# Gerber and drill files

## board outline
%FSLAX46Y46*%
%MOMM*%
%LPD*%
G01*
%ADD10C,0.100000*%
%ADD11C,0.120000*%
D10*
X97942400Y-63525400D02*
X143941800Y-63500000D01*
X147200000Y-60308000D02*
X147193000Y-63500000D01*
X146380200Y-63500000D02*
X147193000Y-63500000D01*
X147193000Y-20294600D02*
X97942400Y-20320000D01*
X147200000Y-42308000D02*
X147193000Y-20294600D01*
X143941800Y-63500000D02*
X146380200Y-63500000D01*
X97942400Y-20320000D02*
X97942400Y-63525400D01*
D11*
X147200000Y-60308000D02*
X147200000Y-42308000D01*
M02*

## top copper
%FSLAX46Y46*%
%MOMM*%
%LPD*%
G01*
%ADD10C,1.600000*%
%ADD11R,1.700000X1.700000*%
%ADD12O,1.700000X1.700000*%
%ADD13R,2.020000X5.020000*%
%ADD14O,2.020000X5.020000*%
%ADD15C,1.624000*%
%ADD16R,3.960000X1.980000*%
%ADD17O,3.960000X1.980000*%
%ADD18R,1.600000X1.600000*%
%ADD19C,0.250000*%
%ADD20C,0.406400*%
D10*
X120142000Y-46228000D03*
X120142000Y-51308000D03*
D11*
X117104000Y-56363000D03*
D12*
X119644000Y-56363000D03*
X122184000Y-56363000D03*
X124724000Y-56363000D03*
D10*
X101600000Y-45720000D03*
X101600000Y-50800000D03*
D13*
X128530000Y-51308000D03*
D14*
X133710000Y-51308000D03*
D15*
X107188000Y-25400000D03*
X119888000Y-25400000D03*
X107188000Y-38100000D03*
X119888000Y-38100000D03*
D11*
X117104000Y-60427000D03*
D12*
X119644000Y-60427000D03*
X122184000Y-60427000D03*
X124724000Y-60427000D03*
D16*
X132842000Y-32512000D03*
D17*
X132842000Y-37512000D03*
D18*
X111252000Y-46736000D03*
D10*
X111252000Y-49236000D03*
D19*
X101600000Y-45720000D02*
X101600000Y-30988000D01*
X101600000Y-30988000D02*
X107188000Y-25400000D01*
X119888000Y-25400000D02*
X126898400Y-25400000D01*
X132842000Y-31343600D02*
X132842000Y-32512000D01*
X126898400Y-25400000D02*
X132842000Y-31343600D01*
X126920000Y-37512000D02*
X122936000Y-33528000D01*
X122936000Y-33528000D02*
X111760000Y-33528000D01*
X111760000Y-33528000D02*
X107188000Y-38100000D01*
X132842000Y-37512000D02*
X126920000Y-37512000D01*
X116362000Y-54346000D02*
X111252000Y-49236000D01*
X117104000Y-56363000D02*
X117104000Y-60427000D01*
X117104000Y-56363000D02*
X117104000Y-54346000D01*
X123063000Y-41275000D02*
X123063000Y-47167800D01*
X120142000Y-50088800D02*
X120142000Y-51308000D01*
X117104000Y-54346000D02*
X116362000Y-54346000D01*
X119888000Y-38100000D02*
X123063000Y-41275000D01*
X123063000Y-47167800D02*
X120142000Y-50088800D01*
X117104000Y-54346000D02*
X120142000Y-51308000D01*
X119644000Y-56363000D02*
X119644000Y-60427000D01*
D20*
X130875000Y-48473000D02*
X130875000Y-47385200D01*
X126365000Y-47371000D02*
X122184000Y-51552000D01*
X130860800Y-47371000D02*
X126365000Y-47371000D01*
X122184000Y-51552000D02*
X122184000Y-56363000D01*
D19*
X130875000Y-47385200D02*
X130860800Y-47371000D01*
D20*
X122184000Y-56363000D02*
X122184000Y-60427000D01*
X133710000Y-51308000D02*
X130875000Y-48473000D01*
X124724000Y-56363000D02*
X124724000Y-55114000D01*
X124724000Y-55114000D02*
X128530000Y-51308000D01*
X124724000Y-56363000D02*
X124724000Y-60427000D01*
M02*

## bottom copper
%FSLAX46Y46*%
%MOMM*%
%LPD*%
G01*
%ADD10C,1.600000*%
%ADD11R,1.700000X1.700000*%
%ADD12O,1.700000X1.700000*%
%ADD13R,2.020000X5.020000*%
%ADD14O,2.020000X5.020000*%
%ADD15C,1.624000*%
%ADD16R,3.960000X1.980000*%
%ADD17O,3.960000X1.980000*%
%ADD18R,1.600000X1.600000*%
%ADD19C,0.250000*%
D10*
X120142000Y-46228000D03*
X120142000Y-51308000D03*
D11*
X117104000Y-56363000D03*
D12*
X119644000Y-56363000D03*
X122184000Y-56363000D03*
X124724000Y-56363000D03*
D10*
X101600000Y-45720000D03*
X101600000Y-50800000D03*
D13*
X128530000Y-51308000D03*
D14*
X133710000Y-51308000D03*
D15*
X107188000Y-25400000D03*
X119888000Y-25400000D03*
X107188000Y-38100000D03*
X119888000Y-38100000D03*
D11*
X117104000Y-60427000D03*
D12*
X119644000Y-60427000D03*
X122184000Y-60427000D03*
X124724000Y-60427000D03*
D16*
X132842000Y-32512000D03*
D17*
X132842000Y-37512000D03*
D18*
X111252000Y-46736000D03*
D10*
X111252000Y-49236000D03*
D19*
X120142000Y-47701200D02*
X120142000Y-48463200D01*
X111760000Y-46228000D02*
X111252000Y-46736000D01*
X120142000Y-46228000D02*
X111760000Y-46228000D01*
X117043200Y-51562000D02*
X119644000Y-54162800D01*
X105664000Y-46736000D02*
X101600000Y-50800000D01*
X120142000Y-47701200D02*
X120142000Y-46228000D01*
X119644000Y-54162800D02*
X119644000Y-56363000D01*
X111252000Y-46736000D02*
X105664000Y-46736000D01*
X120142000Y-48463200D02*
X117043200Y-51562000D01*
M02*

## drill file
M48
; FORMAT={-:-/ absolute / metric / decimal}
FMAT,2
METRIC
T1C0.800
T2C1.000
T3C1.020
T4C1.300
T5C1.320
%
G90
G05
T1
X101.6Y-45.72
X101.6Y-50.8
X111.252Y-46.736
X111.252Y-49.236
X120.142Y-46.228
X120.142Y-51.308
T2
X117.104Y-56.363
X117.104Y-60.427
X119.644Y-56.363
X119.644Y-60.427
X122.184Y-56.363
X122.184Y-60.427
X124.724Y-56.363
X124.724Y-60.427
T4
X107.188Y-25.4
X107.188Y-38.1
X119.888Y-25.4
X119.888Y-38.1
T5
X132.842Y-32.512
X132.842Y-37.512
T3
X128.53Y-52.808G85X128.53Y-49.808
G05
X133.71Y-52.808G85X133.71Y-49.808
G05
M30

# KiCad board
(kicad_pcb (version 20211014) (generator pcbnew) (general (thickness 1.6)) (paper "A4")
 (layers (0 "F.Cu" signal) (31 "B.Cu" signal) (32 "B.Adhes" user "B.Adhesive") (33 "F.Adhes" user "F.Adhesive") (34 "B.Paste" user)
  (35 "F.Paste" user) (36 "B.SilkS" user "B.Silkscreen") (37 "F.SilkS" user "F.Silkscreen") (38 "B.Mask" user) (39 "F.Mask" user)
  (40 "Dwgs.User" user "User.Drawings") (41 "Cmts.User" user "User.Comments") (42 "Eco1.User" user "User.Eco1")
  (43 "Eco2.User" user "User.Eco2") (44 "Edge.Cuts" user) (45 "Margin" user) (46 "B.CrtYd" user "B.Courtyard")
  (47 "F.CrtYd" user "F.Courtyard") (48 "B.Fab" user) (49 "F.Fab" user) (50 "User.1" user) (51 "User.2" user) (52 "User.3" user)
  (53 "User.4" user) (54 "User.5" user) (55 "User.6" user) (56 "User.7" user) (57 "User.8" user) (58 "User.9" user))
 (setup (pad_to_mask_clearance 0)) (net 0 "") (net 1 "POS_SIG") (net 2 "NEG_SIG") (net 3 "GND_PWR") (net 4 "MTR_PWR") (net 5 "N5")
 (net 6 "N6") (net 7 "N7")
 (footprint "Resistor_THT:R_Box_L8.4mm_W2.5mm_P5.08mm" (layer "F.Cu") (at 120.142 46.228 -90)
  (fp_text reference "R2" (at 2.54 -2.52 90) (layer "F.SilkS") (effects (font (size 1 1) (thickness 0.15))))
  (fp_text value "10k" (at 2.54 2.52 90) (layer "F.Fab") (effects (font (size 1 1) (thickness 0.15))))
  (pad "1" thru_hole circle (at 0 0 270) (size 1.6 1.6) (drill 0.8) (layers *.Cu *.Mask) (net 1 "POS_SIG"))
  (pad "2" thru_hole circle (at 5.08 0 270) (size 1.6 1.6) (drill 0.8) (layers *.Cu *.Mask) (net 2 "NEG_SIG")))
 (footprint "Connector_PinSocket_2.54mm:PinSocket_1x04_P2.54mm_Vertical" (layer "F.Cu") (at 117.104 56.363 90)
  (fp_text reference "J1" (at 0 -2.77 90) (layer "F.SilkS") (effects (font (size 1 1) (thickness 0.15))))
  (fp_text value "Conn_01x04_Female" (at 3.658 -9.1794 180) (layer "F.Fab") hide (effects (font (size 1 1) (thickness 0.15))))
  (pad "1" thru_hole rect (at 0 0 90) (size 1.7 1.7) (drill 1) (layers *.Cu *.Mask) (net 2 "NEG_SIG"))
  (pad "2" thru_hole oval (at 0 2.54 90) (size 1.7 1.7) (drill 1) (layers *.Cu *.Mask) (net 1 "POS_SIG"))
  (pad "3" thru_hole oval (at 0 5.08 90) (size 1.7 1.7) (drill 1) (layers *.Cu *.Mask) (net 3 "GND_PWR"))
  (pad "4" thru_hole oval (at 0 7.62 90) (size 1.7 1.7) (drill 1) (layers *.Cu *.Mask) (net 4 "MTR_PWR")))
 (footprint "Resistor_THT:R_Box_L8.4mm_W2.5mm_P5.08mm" (layer "F.Cu") (at 101.6 45.72 -90)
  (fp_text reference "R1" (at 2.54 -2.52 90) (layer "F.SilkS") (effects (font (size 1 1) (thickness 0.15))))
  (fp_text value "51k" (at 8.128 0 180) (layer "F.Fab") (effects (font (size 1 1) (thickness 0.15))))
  (pad "1" thru_hole circle (at 0 0 270) (size 1.6 1.6) (drill 0.8) (layers *.Cu *.Mask) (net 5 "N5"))
  (pad "2" thru_hole circle (at 5.08 0 270) (size 1.6 1.6) (drill 0.8) (layers *.Cu *.Mask) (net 1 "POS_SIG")))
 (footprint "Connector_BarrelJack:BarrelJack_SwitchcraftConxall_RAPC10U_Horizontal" (layer "F.Cu") (at 128.53 51.308 180)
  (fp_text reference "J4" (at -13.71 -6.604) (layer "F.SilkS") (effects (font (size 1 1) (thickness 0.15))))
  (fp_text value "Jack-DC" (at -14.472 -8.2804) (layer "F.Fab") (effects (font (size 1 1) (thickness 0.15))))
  (fp_line (start -18.67 -9) (end -18.67 9) (layer "Edge.Cuts") (width 0.12))
  (pad "1" thru_hole rect (at 0 0 180) (size 2.02 5.02) (drill oval 1.02 4.02) (layers *.Cu *.Mask) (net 4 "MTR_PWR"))
  (pad "2" thru_hole oval (at -5.18 0 180) (size 2.02 5.02) (drill oval 1.02 4.02) (layers *.Cu *.Mask) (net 3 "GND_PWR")))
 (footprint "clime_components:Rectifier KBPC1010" (layer "F.Cu") (at 107.188 25.4)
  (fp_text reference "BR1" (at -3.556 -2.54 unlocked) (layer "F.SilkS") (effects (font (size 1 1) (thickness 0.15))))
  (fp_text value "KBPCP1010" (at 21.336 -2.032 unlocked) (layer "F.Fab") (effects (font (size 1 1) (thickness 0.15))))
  (pad "1" thru_hole circle (at 0 0) (size 1.624 1.624) (drill 1.3) (layers *.Cu *.Mask) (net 5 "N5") (clearance 1))
  (pad "2" thru_hole circle (at 12.7 0) (size 1.624 1.624) (drill 1.3) (layers *.Cu *.Mask) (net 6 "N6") (clearance 1))
  (pad "3" thru_hole circle (at 0 12.7) (size 1.624 1.624) (drill 1.3) (layers *.Cu *.Mask) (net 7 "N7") (clearance 1))
  (pad "4" thru_hole circle (at 12.7 12.7) (size 1.624 1.624) (drill 1.3) (layers *.Cu *.Mask) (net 2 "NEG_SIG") (clearance 1)))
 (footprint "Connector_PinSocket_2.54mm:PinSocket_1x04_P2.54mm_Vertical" (layer "F.Cu") (at 117.104 60.427 90)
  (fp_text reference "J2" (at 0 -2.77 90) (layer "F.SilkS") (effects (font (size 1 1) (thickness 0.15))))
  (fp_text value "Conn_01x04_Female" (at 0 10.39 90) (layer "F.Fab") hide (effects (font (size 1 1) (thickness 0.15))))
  (pad "1" thru_hole rect (at 0 0 90) (size 1.7 1.7) (drill 1) (layers *.Cu *.Mask) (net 2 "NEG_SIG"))
  (pad "2" thru_hole oval (at 0 2.54 90) (size 1.7 1.7) (drill 1) (layers *.Cu *.Mask) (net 1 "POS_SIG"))
  (pad "3" thru_hole oval (at 0 5.08 90) (size 1.7 1.7) (drill 1) (layers *.Cu *.Mask) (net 3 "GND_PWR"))
  (pad "4" thru_hole oval (at 0 7.62 90) (size 1.7 1.7) (drill 1) (layers *.Cu *.Mask) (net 4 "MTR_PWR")))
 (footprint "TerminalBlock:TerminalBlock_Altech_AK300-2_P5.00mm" (layer "F.Cu") (at 132.842 32.512 -90)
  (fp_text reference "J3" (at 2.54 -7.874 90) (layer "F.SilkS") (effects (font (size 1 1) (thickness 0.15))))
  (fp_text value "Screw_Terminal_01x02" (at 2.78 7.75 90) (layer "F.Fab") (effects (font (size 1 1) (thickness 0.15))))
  (pad "1" thru_hole rect (at 0 0 270) (size 1.98 3.96) (drill 1.32) (layers *.Cu *.Mask) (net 6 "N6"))
  (pad "2" thru_hole oval (at 5 0 270) (size 1.98 3.96) (drill 1.32) (layers *.Cu *.Mask) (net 7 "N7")))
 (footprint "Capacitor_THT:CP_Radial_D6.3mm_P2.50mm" (layer "F.Cu") (at 111.252 46.736 -90)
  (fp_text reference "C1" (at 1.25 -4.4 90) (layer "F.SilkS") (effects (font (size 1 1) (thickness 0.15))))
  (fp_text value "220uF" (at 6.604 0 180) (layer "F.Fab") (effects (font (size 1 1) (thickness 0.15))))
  (pad "1" thru_hole rect (at 0 0 270) (size 1.6 1.6) (drill 0.8) (layers *.Cu *.Mask) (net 1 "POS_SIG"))
  (pad "2" thru_hole circle (at 2.5 0 270) (size 1.6 1.6) (drill 0.8) (layers *.Cu *.Mask) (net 2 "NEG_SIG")))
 (gr_line (start 97.9424 63.5254) (end 143.9418 63.5) (layer "Edge.Cuts") (width 0.1))
 (gr_line (start 147.2 60.308) (end 147.193 63.5) (layer "Edge.Cuts") (width 0.1))
 (gr_line (start 146.3802 63.5) (end 147.193 63.5) (layer "Edge.Cuts") (width 0.1))
 (gr_line (start 147.193 20.2946) (end 97.9424 20.32) (layer "Edge.Cuts") (width 0.1))
 (gr_line (start 147.2 42.308) (end 147.193 20.2946) (layer "Edge.Cuts") (width 0.1))
 (gr_line (start 143.9418 63.5) (end 146.3802 63.5) (layer "Edge.Cuts") (width 0.1))
 (gr_line (start 97.9424 20.32) (end 97.9424 63.5254) (layer "Edge.Cuts") (width 0.1))
 (segment (start 101.6 45.72) (end 101.6 30.988) (width 0.25) (layer "F.Cu") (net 5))
 (segment (start 101.6 30.988) (end 107.188 25.4) (width 0.25) (layer "F.Cu") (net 5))
 (segment (start 119.888 25.4) (end 126.8984 25.4) (width 0.25) (layer "F.Cu") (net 6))
 (segment (start 132.842 31.3436) (end 132.842 32.512) (width 0.25) (layer "F.Cu") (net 6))
 (segment (start 126.8984 25.4) (end 132.842 31.3436) (width 0.25) (layer "F.Cu") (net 6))
 (segment (start 126.92 37.512) (end 122.936 33.528) (width 0.25) (layer "F.Cu") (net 7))
 (segment (start 122.936 33.528) (end 111.76 33.528) (width 0.25) (layer "F.Cu") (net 7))
 (segment (start 111.76 33.528) (end 107.188 38.1) (width 0.25) (layer "F.Cu") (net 7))
 (segment (start 132.842 37.512) (end 126.92 37.512) (width 0.25) (layer "F.Cu") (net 7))
 (segment (start 116.362 54.346) (end 111.252 49.236) (width 0.25) (layer "F.Cu") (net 2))
 (segment (start 117.104 56.363) (end 117.104 60.427) (width 0.25) (layer "F.Cu") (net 2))
 (segment (start 117.104 56.363) (end 117.104 54.346) (width 0.25) (layer "F.Cu") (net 2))
 (segment (start 123.063 41.275) (end 123.063 47.1678) (width 0.25) (layer "F.Cu") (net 2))
 (segment (start 120.142 50.0888) (end 120.142 51.308) (width 0.25) (layer "F.Cu") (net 2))
 (segment (start 117.104 54.346) (end 116.362 54.346) (width 0.25) (layer "F.Cu") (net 2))
 (segment (start 119.888 38.1) (end 123.063 41.275) (width 0.25) (layer "F.Cu") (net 2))
 (segment (start 123.063 47.1678) (end 120.142 50.0888) (width 0.25) (layer "F.Cu") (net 2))
 (segment (start 117.104 54.346) (end 120.142 51.308) (width 0.25) (layer "F.Cu") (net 2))
 (segment (start 119.644 56.363) (end 119.644 60.427) (width 0.25) (layer "F.Cu") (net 1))
 (segment (start 120.142 47.7012) (end 120.142 48.4632) (width 0.25) (layer "B.Cu") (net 1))
 (segment (start 111.76 46.228) (end 111.252 46.736) (width 0.25) (layer "B.Cu") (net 1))
 (segment (start 120.142 46.228) (end 111.76 46.228) (width 0.25) (layer "B.Cu") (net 1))
 (segment (start 117.0432 51.562) (end 119.644 54.1628) (width 0.25) (layer "B.Cu") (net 1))
 (segment (start 105.664 46.736) (end 101.6 50.8) (width 0.25) (layer "B.Cu") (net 1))
 (segment (start 120.142 47.7012) (end 120.142 46.228) (width 0.25) (layer "B.Cu") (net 1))
 (segment (start 119.644 54.1628) (end 119.644 56.363) (width 0.25) (layer "B.Cu") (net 1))
 (segment (start 111.252 46.736) (end 105.664 46.736) (width 0.25) (layer "B.Cu") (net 1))
 (segment (start 120.142 48.4632) (end 117.0432 51.562) (width 0.25) (layer "B.Cu") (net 1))
 (segment (start 130.875 48.473) (end 130.875 47.3852) (width 0.4064) (layer "F.Cu") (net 3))
 (segment (start 126.365 47.371) (end 122.184 51.552) (width 0.4064) (layer "F.Cu") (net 3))
 (segment (start 130.8608 47.371) (end 126.365 47.371) (width 0.4064) (layer "F.Cu") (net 3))
 (segment (start 122.184 51.552) (end 122.184 56.363) (width 0.4064) (layer "F.Cu") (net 3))
 (segment (start 130.875 47.3852) (end 130.8608 47.371) (width 0.25) (layer "F.Cu") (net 3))
 (segment (start 122.184 56.363) (end 122.184 60.427) (width 0.4064) (layer "F.Cu") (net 3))
 (segment (start 133.71 51.308) (end 130.875 48.473) (width 0.4064) (layer "F.Cu") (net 3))
 (segment (start 124.724 56.363) (end 124.724 55.114) (width 0.4064) (layer "F.Cu") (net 4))
 (segment (start 124.724 55.114) (end 128.53 51.308) (width 0.4064) (layer "F.Cu") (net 4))
 (segment (start 124.724 56.363) (end 124.724 60.427) (width 0.4064) (layer "F.Cu") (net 4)))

